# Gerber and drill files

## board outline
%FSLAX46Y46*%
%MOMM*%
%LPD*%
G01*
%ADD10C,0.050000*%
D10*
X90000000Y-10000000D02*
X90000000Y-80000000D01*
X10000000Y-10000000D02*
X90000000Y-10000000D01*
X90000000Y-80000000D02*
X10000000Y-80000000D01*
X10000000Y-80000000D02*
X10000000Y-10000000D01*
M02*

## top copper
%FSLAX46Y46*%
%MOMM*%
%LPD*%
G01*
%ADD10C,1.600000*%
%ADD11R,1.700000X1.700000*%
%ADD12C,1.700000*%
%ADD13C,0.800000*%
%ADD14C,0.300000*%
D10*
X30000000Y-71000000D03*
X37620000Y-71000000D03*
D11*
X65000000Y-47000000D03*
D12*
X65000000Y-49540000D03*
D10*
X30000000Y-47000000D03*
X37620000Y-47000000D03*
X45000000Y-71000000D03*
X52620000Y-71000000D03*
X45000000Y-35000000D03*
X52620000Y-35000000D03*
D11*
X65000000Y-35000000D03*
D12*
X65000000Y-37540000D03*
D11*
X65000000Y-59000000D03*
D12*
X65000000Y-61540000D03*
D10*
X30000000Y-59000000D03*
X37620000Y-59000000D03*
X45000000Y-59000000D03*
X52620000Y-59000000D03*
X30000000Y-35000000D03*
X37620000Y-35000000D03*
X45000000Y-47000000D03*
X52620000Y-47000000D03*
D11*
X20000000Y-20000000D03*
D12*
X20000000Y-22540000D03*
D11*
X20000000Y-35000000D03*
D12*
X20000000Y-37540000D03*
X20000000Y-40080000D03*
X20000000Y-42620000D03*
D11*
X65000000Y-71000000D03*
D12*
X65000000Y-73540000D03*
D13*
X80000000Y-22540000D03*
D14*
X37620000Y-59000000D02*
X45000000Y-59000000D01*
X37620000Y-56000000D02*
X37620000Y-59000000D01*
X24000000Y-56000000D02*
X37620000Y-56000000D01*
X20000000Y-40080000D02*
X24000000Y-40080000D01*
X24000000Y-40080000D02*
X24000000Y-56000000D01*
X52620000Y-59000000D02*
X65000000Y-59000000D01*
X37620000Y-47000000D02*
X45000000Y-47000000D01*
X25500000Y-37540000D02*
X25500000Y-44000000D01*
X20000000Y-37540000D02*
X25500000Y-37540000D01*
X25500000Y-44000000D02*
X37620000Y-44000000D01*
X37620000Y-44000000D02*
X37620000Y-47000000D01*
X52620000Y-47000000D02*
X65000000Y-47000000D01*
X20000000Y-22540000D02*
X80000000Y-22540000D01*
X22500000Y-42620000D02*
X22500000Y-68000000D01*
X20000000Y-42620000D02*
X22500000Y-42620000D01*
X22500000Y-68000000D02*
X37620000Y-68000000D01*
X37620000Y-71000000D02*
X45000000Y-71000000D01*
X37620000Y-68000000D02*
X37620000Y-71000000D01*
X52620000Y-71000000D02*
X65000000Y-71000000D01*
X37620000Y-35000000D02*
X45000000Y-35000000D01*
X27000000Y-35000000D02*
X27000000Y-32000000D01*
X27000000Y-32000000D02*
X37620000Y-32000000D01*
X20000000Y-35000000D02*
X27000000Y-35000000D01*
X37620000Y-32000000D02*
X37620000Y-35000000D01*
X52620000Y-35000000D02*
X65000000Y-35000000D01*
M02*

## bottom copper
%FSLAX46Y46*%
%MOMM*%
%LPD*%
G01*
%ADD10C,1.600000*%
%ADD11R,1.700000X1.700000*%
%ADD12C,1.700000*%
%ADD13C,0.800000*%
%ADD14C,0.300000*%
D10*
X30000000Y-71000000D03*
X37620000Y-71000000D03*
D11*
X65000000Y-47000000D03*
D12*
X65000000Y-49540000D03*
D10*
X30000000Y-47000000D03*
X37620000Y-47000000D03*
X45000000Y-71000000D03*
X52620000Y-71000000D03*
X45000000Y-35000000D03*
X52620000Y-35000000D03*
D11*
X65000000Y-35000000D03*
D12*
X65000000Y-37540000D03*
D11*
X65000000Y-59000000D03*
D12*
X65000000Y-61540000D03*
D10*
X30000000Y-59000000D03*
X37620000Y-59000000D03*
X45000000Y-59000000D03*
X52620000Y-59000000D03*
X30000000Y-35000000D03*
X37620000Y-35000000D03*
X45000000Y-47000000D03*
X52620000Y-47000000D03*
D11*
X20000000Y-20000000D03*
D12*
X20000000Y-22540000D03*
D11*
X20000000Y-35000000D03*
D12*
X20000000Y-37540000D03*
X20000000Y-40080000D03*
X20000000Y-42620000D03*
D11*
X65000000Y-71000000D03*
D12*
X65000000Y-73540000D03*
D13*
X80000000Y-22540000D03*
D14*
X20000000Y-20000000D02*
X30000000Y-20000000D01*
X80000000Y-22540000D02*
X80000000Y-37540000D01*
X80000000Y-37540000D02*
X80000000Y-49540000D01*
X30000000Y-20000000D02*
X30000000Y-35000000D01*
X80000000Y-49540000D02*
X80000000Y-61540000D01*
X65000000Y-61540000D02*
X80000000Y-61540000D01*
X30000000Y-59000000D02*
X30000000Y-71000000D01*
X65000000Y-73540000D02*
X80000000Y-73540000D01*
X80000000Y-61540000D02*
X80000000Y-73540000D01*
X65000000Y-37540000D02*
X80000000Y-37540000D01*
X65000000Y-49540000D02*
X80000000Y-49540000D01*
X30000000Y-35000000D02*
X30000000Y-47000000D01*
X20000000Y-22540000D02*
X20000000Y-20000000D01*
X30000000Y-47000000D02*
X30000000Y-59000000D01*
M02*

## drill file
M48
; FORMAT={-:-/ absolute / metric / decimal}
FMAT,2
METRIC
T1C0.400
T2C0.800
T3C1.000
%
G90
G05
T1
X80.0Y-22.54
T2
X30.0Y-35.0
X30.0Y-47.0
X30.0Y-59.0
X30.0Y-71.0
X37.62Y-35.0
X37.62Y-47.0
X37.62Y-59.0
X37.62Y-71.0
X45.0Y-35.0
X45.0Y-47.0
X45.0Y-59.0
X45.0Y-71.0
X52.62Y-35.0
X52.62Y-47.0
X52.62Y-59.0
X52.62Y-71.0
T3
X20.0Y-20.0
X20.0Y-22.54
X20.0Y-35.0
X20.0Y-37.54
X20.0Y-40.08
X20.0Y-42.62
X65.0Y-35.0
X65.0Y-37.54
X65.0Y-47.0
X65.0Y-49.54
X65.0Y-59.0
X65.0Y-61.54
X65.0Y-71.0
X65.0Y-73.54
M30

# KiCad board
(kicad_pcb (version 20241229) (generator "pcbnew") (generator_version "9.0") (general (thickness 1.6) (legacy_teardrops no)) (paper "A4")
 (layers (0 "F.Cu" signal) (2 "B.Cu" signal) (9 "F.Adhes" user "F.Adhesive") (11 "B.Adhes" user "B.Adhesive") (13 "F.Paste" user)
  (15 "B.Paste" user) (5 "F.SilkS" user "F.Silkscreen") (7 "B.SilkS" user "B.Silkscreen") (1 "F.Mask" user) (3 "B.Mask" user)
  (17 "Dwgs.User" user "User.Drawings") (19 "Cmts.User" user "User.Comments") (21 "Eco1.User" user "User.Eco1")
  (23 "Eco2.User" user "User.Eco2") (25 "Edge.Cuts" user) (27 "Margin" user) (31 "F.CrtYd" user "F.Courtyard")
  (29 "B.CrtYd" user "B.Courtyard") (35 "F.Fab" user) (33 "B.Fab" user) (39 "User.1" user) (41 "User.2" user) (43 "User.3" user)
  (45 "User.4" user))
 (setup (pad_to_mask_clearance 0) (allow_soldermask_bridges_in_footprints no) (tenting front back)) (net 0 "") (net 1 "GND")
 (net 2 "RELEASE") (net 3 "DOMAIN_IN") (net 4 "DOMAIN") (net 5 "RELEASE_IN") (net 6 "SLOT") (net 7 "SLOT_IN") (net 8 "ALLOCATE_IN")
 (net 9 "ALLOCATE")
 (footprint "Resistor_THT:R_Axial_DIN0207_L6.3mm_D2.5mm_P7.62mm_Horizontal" (layer "F.Cu") (at 30 71)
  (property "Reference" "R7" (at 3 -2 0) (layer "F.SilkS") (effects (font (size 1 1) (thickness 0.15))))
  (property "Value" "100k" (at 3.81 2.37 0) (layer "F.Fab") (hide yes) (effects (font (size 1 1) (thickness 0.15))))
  (pad "1" thru_hole circle (at 0 0) (size 1.6 1.6) (drill 0.8) (layers "*.Cu" "*.Mask") (remove_unused_layers no) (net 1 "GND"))
  (pad "2" thru_hole circle (at 7.62 0) (size 1.6 1.6) (drill 0.8) (layers "*.Cu" "*.Mask") (remove_unused_layers no) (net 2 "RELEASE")))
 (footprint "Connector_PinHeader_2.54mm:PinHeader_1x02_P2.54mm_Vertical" (layer "F.Cu") (at 65 47)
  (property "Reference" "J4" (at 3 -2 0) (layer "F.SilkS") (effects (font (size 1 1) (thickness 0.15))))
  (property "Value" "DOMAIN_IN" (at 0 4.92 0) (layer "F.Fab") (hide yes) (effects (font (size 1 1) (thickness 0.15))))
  (pad "1" thru_hole rect (at 0 0) (size 1.7 1.7) (drill 1) (layers "*.Cu" "*.Mask") (remove_unused_layers no) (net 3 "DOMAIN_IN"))
  (pad "2" thru_hole circle (at 0 2.54) (size 1.7 1.7) (drill 1) (layers "*.Cu" "*.Mask") (remove_unused_layers no) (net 1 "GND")))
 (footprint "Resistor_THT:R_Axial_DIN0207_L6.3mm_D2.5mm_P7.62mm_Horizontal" (layer "F.Cu") (at 30 47)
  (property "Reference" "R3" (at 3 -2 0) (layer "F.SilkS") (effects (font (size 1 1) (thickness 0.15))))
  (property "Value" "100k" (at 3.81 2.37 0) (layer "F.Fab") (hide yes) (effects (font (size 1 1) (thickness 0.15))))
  (pad "1" thru_hole circle (at 0 0) (size 1.6 1.6) (drill 0.8) (layers "*.Cu" "*.Mask") (remove_unused_layers no) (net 1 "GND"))
  (pad "2" thru_hole circle (at 7.62 0) (size 1.6 1.6) (drill 0.8) (layers "*.Cu" "*.Mask") (remove_unused_layers no) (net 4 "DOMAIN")))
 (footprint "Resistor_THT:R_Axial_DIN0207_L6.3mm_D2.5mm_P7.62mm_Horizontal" (layer "F.Cu") (at 45 71)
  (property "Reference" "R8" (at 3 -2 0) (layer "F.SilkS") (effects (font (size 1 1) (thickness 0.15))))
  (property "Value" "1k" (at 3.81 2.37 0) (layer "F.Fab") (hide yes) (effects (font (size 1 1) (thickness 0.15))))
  (pad "1" thru_hole circle (at 0 0) (size 1.6 1.6) (drill 0.8) (layers "*.Cu" "*.Mask") (remove_unused_layers no) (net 2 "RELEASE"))
  (pad "2" thru_hole circle (at 7.62 0) (size 1.6 1.6) (drill 0.8) (layers "*.Cu" "*.Mask") (remove_unused_layers no) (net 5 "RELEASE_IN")))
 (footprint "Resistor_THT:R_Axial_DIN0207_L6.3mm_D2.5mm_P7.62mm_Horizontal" (layer "F.Cu") (at 45 35)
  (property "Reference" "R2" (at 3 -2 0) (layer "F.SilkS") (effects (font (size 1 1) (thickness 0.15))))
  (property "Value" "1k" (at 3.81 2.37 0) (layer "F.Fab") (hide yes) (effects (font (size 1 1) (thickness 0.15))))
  (pad "1" thru_hole circle (at 0 0) (size 1.6 1.6) (drill 0.8) (layers "*.Cu" "*.Mask") (remove_unused_layers no) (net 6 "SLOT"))
  (pad "2" thru_hole circle (at 7.62 0) (size 1.6 1.6) (drill 0.8) (layers "*.Cu" "*.Mask") (remove_unused_layers no) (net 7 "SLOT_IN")))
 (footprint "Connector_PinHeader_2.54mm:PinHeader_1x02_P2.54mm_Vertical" (layer "F.Cu") (at 65 35)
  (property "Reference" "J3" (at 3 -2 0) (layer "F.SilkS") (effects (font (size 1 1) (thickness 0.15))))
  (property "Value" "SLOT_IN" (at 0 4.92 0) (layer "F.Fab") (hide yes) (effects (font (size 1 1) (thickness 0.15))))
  (pad "1" thru_hole rect (at 0 0) (size 1.7 1.7) (drill 1) (layers "*.Cu" "*.Mask") (remove_unused_layers no) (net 7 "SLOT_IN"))
  (pad "2" thru_hole circle (at 0 2.54) (size 1.7 1.7) (drill 1) (layers "*.Cu" "*.Mask") (remove_unused_layers no) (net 1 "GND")))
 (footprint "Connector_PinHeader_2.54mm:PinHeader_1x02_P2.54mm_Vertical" (layer "F.Cu") (at 65 59)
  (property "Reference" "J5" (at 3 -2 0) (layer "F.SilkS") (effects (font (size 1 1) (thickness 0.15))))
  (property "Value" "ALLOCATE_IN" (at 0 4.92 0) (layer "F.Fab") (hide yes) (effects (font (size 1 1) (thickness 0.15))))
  (pad "1" thru_hole rect (at 0 0) (size 1.7 1.7) (drill 1) (layers "*.Cu" "*.Mask") (remove_unused_layers no) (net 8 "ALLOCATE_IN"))
  (pad "2" thru_hole circle (at 0 2.54) (size 1.7 1.7) (drill 1) (layers "*.Cu" "*.Mask") (remove_unused_layers no) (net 1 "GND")))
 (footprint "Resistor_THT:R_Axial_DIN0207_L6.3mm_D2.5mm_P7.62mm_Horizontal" (layer "F.Cu") (at 30 59)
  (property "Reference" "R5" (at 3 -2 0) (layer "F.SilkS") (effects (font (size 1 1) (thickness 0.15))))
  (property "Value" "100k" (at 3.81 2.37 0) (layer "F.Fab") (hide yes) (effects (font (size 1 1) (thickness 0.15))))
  (pad "1" thru_hole circle (at 0 0) (size 1.6 1.6) (drill 0.8) (layers "*.Cu" "*.Mask") (remove_unused_layers no) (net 1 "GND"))
  (pad "2" thru_hole circle (at 7.62 0) (size 1.6 1.6) (drill 0.8) (layers "*.Cu" "*.Mask") (remove_unused_layers no) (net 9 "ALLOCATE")))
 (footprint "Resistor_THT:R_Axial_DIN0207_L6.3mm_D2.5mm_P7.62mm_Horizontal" (layer "F.Cu") (at 45 59)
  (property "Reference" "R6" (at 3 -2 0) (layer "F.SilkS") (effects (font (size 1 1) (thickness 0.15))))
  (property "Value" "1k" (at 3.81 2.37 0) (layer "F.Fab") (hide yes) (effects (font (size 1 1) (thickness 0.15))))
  (pad "1" thru_hole circle (at 0 0) (size 1.6 1.6) (drill 0.8) (layers "*.Cu" "*.Mask") (remove_unused_layers no) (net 9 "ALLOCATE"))
  (pad "2" thru_hole circle (at 7.62 0) (size 1.6 1.6) (drill 0.8) (layers "*.Cu" "*.Mask") (remove_unused_layers no) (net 8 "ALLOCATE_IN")))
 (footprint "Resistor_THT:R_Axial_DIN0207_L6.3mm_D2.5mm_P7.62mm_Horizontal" (layer "F.Cu") (at 30 35)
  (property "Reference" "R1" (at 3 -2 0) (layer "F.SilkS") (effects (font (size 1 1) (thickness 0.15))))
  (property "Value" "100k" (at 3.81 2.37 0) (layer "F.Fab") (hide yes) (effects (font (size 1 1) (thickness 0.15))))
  (pad "1" thru_hole circle (at 0 0) (size 1.6 1.6) (drill 0.8) (layers "*.Cu" "*.Mask") (remove_unused_layers no) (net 1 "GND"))
  (pad "2" thru_hole circle (at 7.62 0) (size 1.6 1.6) (drill 0.8) (layers "*.Cu" "*.Mask") (remove_unused_layers no) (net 6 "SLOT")))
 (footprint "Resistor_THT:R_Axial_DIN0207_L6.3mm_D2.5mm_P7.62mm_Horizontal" (layer "F.Cu") (at 45 47)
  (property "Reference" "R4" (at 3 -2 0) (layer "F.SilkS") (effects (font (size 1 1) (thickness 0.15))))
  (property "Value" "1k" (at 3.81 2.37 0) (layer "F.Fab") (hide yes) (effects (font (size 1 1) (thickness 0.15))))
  (pad "1" thru_hole circle (at 0 0) (size 1.6 1.6) (drill 0.8) (layers "*.Cu" "*.Mask") (remove_unused_layers no) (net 4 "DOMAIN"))
  (pad "2" thru_hole circle (at 7.62 0) (size 1.6 1.6) (drill 0.8) (layers "*.Cu" "*.Mask") (remove_unused_layers no) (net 3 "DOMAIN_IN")))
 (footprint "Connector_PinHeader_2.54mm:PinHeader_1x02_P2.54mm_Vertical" (layer "F.Cu") (at 20 20)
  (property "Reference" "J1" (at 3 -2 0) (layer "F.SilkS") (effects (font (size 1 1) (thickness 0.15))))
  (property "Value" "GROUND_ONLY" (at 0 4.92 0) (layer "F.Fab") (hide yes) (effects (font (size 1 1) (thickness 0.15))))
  (pad "1" thru_hole rect (at 0 0) (size 1.7 1.7) (drill 1) (layers "*.Cu" "*.Mask") (remove_unused_layers no) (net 1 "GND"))
  (pad "2" thru_hole circle (at 0 2.54) (size 1.7 1.7) (drill 1) (layers "*.Cu" "*.Mask") (remove_unused_layers no) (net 1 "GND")))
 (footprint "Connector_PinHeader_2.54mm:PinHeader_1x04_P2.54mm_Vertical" (layer "F.Cu") (at 20 35)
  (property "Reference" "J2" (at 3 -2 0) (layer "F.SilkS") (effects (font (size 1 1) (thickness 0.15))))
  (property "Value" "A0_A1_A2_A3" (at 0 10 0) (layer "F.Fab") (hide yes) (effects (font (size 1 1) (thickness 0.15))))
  (pad "1" thru_hole rect (at 0 0) (size 1.7 1.7) (drill 1) (layers "*.Cu" "*.Mask") (remove_unused_layers no) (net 6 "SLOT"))
  (pad "2" thru_hole circle (at 0 2.54) (size 1.7 1.7) (drill 1) (layers "*.Cu" "*.Mask") (remove_unused_layers no) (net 4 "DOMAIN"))
  (pad "3" thru_hole circle (at 0 5.08) (size 1.7 1.7) (drill 1) (layers "*.Cu" "*.Mask") (remove_unused_layers no) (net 9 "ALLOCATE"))
  (pad "4" thru_hole circle (at 0 7.62) (size 1.7 1.7) (drill 1) (layers "*.Cu" "*.Mask") (remove_unused_layers no) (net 2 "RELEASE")))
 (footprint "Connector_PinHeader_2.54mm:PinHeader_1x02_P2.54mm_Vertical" (layer "F.Cu") (at 65 71)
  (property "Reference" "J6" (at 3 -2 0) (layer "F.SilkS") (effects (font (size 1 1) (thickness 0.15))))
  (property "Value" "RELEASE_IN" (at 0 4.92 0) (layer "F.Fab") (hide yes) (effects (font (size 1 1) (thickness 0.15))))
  (pad "1" thru_hole rect (at 0 0) (size 1.7 1.7) (drill 1) (layers "*.Cu" "*.Mask") (remove_unused_layers no) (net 5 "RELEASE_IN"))
  (pad "2" thru_hole circle (at 0 2.54) (size 1.7 1.7) (drill 1) (layers "*.Cu" "*.Mask") (remove_unused_layers no) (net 1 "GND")))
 (gr_line (start 90 10) (end 90 80) (stroke (width 0.05) (type default)) (layer "Edge.Cuts"))
 (gr_line (start 10 10) (end 90 10) (stroke (width 0.05) (type default)) (layer "Edge.Cuts"))
 (gr_line (start 90 80) (end 10 80) (stroke (width 0.05) (type default)) (layer "Edge.Cuts"))
 (gr_line (start 10 80) (end 10 10) (stroke (width 0.05) (type default)) (layer "Edge.Cuts"))
 (segment (start 37.62 59) (end 45 59) (width 0.3) (layer "F.Cu") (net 9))
 (segment (start 37.62 56) (end 37.62 59) (width 0.3) (layer "F.Cu") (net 9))
 (segment (start 24 56) (end 37.62 56) (width 0.3) (layer "F.Cu") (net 9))
 (segment (start 20 40.08) (end 24 40.08) (width 0.3) (layer "F.Cu") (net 9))
 (segment (start 24 40.08) (end 24 56) (width 0.3) (layer "F.Cu") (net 9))
 (segment (start 52.62 59) (end 65 59) (width 0.3) (layer "F.Cu") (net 8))
 (segment (start 37.62 47) (end 45 47) (width 0.3) (layer "F.Cu") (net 4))
 (segment (start 25.5 37.54) (end 25.5 44) (width 0.3) (layer "F.Cu") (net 4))
 (segment (start 20 37.54) (end 25.5 37.54) (width 0.3) (layer "F.Cu") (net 4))
 (segment (start 25.5 44) (end 37.62 44) (width 0.3) (layer "F.Cu") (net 4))
 (segment (start 37.62 44) (end 37.62 47) (width 0.3) (layer "F.Cu") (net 4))
 (segment (start 52.62 47) (end 65 47) (width 0.3) (layer "F.Cu") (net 3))
 (segment (start 20 22.54) (end 80 22.54) (width 0.3) (layer "F.Cu") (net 1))
 (via (at 80 22.54) (size 0.8) (drill 0.4) (layers "F.Cu" "B.Cu") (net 1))
 (segment (start 20 20) (end 30 20) (width 0.3) (layer "B.Cu") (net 1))
 (segment (start 80 22.54) (end 80 37.54) (width 0.3) (layer "B.Cu") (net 1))
 (segment (start 80 37.54) (end 80 49.54) (width 0.3) (layer "B.Cu") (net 1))
 (segment (start 30 20) (end 30 35) (width 0.3) (layer "B.Cu") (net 1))
 (segment (start 80 49.54) (end 80 61.54) (width 0.3) (layer "B.Cu") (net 1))
 (segment (start 65 61.54) (end 80 61.54) (width 0.3) (layer "B.Cu") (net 1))
 (segment (start 30 59) (end 30 71) (width 0.3) (layer "B.Cu") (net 1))
 (segment (start 65 73.54) (end 80 73.54) (width 0.3) (layer "B.Cu") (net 1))
 (segment (start 80 61.54) (end 80 73.54) (width 0.3) (layer "B.Cu") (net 1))
 (segment (start 65 37.54) (end 80 37.54) (width 0.3) (layer "B.Cu") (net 1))
 (segment (start 65 49.54) (end 80 49.54) (width 0.3) (layer "B.Cu") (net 1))
 (segment (start 30 35) (end 30 47) (width 0.3) (layer "B.Cu") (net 1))
 (segment (start 20 22.54) (end 20 20) (width 0.3) (layer "B.Cu") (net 1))
 (segment (start 30 47) (end 30 59) (width 0.3) (layer "B.Cu") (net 1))
 (segment (start 22.5 42.62) (end 22.5 68) (width 0.3) (layer "F.Cu") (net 2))
 (segment (start 20 42.62) (end 22.5 42.62) (width 0.3) (layer "F.Cu") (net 2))
 (segment (start 22.5 68) (end 37.62 68) (width 0.3) (layer "F.Cu") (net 2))
 (segment (start 37.62 71) (end 45 71) (width 0.3) (layer "F.Cu") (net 2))
 (segment (start 37.62 68) (end 37.62 71) (width 0.3) (layer "F.Cu") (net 2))
 (segment (start 52.62 71) (end 65 71) (width 0.3) (layer "F.Cu") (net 5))
 (segment (start 37.62 35) (end 45 35) (width 0.3) (layer "F.Cu") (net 6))
 (segment (start 27 35) (end 27 32) (width 0.3) (layer "F.Cu") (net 6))
 (segment (start 27 32) (end 37.62 32) (width 0.3) (layer "F.Cu") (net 6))
 (segment (start 20 35) (end 27 35) (width 0.3) (layer "F.Cu") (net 6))
 (segment (start 37.62 32) (end 37.62 35) (width 0.3) (layer "F.Cu") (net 6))
 (segment (start 52.62 35) (end 65 35) (width 0.3) (layer "F.Cu") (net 7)))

